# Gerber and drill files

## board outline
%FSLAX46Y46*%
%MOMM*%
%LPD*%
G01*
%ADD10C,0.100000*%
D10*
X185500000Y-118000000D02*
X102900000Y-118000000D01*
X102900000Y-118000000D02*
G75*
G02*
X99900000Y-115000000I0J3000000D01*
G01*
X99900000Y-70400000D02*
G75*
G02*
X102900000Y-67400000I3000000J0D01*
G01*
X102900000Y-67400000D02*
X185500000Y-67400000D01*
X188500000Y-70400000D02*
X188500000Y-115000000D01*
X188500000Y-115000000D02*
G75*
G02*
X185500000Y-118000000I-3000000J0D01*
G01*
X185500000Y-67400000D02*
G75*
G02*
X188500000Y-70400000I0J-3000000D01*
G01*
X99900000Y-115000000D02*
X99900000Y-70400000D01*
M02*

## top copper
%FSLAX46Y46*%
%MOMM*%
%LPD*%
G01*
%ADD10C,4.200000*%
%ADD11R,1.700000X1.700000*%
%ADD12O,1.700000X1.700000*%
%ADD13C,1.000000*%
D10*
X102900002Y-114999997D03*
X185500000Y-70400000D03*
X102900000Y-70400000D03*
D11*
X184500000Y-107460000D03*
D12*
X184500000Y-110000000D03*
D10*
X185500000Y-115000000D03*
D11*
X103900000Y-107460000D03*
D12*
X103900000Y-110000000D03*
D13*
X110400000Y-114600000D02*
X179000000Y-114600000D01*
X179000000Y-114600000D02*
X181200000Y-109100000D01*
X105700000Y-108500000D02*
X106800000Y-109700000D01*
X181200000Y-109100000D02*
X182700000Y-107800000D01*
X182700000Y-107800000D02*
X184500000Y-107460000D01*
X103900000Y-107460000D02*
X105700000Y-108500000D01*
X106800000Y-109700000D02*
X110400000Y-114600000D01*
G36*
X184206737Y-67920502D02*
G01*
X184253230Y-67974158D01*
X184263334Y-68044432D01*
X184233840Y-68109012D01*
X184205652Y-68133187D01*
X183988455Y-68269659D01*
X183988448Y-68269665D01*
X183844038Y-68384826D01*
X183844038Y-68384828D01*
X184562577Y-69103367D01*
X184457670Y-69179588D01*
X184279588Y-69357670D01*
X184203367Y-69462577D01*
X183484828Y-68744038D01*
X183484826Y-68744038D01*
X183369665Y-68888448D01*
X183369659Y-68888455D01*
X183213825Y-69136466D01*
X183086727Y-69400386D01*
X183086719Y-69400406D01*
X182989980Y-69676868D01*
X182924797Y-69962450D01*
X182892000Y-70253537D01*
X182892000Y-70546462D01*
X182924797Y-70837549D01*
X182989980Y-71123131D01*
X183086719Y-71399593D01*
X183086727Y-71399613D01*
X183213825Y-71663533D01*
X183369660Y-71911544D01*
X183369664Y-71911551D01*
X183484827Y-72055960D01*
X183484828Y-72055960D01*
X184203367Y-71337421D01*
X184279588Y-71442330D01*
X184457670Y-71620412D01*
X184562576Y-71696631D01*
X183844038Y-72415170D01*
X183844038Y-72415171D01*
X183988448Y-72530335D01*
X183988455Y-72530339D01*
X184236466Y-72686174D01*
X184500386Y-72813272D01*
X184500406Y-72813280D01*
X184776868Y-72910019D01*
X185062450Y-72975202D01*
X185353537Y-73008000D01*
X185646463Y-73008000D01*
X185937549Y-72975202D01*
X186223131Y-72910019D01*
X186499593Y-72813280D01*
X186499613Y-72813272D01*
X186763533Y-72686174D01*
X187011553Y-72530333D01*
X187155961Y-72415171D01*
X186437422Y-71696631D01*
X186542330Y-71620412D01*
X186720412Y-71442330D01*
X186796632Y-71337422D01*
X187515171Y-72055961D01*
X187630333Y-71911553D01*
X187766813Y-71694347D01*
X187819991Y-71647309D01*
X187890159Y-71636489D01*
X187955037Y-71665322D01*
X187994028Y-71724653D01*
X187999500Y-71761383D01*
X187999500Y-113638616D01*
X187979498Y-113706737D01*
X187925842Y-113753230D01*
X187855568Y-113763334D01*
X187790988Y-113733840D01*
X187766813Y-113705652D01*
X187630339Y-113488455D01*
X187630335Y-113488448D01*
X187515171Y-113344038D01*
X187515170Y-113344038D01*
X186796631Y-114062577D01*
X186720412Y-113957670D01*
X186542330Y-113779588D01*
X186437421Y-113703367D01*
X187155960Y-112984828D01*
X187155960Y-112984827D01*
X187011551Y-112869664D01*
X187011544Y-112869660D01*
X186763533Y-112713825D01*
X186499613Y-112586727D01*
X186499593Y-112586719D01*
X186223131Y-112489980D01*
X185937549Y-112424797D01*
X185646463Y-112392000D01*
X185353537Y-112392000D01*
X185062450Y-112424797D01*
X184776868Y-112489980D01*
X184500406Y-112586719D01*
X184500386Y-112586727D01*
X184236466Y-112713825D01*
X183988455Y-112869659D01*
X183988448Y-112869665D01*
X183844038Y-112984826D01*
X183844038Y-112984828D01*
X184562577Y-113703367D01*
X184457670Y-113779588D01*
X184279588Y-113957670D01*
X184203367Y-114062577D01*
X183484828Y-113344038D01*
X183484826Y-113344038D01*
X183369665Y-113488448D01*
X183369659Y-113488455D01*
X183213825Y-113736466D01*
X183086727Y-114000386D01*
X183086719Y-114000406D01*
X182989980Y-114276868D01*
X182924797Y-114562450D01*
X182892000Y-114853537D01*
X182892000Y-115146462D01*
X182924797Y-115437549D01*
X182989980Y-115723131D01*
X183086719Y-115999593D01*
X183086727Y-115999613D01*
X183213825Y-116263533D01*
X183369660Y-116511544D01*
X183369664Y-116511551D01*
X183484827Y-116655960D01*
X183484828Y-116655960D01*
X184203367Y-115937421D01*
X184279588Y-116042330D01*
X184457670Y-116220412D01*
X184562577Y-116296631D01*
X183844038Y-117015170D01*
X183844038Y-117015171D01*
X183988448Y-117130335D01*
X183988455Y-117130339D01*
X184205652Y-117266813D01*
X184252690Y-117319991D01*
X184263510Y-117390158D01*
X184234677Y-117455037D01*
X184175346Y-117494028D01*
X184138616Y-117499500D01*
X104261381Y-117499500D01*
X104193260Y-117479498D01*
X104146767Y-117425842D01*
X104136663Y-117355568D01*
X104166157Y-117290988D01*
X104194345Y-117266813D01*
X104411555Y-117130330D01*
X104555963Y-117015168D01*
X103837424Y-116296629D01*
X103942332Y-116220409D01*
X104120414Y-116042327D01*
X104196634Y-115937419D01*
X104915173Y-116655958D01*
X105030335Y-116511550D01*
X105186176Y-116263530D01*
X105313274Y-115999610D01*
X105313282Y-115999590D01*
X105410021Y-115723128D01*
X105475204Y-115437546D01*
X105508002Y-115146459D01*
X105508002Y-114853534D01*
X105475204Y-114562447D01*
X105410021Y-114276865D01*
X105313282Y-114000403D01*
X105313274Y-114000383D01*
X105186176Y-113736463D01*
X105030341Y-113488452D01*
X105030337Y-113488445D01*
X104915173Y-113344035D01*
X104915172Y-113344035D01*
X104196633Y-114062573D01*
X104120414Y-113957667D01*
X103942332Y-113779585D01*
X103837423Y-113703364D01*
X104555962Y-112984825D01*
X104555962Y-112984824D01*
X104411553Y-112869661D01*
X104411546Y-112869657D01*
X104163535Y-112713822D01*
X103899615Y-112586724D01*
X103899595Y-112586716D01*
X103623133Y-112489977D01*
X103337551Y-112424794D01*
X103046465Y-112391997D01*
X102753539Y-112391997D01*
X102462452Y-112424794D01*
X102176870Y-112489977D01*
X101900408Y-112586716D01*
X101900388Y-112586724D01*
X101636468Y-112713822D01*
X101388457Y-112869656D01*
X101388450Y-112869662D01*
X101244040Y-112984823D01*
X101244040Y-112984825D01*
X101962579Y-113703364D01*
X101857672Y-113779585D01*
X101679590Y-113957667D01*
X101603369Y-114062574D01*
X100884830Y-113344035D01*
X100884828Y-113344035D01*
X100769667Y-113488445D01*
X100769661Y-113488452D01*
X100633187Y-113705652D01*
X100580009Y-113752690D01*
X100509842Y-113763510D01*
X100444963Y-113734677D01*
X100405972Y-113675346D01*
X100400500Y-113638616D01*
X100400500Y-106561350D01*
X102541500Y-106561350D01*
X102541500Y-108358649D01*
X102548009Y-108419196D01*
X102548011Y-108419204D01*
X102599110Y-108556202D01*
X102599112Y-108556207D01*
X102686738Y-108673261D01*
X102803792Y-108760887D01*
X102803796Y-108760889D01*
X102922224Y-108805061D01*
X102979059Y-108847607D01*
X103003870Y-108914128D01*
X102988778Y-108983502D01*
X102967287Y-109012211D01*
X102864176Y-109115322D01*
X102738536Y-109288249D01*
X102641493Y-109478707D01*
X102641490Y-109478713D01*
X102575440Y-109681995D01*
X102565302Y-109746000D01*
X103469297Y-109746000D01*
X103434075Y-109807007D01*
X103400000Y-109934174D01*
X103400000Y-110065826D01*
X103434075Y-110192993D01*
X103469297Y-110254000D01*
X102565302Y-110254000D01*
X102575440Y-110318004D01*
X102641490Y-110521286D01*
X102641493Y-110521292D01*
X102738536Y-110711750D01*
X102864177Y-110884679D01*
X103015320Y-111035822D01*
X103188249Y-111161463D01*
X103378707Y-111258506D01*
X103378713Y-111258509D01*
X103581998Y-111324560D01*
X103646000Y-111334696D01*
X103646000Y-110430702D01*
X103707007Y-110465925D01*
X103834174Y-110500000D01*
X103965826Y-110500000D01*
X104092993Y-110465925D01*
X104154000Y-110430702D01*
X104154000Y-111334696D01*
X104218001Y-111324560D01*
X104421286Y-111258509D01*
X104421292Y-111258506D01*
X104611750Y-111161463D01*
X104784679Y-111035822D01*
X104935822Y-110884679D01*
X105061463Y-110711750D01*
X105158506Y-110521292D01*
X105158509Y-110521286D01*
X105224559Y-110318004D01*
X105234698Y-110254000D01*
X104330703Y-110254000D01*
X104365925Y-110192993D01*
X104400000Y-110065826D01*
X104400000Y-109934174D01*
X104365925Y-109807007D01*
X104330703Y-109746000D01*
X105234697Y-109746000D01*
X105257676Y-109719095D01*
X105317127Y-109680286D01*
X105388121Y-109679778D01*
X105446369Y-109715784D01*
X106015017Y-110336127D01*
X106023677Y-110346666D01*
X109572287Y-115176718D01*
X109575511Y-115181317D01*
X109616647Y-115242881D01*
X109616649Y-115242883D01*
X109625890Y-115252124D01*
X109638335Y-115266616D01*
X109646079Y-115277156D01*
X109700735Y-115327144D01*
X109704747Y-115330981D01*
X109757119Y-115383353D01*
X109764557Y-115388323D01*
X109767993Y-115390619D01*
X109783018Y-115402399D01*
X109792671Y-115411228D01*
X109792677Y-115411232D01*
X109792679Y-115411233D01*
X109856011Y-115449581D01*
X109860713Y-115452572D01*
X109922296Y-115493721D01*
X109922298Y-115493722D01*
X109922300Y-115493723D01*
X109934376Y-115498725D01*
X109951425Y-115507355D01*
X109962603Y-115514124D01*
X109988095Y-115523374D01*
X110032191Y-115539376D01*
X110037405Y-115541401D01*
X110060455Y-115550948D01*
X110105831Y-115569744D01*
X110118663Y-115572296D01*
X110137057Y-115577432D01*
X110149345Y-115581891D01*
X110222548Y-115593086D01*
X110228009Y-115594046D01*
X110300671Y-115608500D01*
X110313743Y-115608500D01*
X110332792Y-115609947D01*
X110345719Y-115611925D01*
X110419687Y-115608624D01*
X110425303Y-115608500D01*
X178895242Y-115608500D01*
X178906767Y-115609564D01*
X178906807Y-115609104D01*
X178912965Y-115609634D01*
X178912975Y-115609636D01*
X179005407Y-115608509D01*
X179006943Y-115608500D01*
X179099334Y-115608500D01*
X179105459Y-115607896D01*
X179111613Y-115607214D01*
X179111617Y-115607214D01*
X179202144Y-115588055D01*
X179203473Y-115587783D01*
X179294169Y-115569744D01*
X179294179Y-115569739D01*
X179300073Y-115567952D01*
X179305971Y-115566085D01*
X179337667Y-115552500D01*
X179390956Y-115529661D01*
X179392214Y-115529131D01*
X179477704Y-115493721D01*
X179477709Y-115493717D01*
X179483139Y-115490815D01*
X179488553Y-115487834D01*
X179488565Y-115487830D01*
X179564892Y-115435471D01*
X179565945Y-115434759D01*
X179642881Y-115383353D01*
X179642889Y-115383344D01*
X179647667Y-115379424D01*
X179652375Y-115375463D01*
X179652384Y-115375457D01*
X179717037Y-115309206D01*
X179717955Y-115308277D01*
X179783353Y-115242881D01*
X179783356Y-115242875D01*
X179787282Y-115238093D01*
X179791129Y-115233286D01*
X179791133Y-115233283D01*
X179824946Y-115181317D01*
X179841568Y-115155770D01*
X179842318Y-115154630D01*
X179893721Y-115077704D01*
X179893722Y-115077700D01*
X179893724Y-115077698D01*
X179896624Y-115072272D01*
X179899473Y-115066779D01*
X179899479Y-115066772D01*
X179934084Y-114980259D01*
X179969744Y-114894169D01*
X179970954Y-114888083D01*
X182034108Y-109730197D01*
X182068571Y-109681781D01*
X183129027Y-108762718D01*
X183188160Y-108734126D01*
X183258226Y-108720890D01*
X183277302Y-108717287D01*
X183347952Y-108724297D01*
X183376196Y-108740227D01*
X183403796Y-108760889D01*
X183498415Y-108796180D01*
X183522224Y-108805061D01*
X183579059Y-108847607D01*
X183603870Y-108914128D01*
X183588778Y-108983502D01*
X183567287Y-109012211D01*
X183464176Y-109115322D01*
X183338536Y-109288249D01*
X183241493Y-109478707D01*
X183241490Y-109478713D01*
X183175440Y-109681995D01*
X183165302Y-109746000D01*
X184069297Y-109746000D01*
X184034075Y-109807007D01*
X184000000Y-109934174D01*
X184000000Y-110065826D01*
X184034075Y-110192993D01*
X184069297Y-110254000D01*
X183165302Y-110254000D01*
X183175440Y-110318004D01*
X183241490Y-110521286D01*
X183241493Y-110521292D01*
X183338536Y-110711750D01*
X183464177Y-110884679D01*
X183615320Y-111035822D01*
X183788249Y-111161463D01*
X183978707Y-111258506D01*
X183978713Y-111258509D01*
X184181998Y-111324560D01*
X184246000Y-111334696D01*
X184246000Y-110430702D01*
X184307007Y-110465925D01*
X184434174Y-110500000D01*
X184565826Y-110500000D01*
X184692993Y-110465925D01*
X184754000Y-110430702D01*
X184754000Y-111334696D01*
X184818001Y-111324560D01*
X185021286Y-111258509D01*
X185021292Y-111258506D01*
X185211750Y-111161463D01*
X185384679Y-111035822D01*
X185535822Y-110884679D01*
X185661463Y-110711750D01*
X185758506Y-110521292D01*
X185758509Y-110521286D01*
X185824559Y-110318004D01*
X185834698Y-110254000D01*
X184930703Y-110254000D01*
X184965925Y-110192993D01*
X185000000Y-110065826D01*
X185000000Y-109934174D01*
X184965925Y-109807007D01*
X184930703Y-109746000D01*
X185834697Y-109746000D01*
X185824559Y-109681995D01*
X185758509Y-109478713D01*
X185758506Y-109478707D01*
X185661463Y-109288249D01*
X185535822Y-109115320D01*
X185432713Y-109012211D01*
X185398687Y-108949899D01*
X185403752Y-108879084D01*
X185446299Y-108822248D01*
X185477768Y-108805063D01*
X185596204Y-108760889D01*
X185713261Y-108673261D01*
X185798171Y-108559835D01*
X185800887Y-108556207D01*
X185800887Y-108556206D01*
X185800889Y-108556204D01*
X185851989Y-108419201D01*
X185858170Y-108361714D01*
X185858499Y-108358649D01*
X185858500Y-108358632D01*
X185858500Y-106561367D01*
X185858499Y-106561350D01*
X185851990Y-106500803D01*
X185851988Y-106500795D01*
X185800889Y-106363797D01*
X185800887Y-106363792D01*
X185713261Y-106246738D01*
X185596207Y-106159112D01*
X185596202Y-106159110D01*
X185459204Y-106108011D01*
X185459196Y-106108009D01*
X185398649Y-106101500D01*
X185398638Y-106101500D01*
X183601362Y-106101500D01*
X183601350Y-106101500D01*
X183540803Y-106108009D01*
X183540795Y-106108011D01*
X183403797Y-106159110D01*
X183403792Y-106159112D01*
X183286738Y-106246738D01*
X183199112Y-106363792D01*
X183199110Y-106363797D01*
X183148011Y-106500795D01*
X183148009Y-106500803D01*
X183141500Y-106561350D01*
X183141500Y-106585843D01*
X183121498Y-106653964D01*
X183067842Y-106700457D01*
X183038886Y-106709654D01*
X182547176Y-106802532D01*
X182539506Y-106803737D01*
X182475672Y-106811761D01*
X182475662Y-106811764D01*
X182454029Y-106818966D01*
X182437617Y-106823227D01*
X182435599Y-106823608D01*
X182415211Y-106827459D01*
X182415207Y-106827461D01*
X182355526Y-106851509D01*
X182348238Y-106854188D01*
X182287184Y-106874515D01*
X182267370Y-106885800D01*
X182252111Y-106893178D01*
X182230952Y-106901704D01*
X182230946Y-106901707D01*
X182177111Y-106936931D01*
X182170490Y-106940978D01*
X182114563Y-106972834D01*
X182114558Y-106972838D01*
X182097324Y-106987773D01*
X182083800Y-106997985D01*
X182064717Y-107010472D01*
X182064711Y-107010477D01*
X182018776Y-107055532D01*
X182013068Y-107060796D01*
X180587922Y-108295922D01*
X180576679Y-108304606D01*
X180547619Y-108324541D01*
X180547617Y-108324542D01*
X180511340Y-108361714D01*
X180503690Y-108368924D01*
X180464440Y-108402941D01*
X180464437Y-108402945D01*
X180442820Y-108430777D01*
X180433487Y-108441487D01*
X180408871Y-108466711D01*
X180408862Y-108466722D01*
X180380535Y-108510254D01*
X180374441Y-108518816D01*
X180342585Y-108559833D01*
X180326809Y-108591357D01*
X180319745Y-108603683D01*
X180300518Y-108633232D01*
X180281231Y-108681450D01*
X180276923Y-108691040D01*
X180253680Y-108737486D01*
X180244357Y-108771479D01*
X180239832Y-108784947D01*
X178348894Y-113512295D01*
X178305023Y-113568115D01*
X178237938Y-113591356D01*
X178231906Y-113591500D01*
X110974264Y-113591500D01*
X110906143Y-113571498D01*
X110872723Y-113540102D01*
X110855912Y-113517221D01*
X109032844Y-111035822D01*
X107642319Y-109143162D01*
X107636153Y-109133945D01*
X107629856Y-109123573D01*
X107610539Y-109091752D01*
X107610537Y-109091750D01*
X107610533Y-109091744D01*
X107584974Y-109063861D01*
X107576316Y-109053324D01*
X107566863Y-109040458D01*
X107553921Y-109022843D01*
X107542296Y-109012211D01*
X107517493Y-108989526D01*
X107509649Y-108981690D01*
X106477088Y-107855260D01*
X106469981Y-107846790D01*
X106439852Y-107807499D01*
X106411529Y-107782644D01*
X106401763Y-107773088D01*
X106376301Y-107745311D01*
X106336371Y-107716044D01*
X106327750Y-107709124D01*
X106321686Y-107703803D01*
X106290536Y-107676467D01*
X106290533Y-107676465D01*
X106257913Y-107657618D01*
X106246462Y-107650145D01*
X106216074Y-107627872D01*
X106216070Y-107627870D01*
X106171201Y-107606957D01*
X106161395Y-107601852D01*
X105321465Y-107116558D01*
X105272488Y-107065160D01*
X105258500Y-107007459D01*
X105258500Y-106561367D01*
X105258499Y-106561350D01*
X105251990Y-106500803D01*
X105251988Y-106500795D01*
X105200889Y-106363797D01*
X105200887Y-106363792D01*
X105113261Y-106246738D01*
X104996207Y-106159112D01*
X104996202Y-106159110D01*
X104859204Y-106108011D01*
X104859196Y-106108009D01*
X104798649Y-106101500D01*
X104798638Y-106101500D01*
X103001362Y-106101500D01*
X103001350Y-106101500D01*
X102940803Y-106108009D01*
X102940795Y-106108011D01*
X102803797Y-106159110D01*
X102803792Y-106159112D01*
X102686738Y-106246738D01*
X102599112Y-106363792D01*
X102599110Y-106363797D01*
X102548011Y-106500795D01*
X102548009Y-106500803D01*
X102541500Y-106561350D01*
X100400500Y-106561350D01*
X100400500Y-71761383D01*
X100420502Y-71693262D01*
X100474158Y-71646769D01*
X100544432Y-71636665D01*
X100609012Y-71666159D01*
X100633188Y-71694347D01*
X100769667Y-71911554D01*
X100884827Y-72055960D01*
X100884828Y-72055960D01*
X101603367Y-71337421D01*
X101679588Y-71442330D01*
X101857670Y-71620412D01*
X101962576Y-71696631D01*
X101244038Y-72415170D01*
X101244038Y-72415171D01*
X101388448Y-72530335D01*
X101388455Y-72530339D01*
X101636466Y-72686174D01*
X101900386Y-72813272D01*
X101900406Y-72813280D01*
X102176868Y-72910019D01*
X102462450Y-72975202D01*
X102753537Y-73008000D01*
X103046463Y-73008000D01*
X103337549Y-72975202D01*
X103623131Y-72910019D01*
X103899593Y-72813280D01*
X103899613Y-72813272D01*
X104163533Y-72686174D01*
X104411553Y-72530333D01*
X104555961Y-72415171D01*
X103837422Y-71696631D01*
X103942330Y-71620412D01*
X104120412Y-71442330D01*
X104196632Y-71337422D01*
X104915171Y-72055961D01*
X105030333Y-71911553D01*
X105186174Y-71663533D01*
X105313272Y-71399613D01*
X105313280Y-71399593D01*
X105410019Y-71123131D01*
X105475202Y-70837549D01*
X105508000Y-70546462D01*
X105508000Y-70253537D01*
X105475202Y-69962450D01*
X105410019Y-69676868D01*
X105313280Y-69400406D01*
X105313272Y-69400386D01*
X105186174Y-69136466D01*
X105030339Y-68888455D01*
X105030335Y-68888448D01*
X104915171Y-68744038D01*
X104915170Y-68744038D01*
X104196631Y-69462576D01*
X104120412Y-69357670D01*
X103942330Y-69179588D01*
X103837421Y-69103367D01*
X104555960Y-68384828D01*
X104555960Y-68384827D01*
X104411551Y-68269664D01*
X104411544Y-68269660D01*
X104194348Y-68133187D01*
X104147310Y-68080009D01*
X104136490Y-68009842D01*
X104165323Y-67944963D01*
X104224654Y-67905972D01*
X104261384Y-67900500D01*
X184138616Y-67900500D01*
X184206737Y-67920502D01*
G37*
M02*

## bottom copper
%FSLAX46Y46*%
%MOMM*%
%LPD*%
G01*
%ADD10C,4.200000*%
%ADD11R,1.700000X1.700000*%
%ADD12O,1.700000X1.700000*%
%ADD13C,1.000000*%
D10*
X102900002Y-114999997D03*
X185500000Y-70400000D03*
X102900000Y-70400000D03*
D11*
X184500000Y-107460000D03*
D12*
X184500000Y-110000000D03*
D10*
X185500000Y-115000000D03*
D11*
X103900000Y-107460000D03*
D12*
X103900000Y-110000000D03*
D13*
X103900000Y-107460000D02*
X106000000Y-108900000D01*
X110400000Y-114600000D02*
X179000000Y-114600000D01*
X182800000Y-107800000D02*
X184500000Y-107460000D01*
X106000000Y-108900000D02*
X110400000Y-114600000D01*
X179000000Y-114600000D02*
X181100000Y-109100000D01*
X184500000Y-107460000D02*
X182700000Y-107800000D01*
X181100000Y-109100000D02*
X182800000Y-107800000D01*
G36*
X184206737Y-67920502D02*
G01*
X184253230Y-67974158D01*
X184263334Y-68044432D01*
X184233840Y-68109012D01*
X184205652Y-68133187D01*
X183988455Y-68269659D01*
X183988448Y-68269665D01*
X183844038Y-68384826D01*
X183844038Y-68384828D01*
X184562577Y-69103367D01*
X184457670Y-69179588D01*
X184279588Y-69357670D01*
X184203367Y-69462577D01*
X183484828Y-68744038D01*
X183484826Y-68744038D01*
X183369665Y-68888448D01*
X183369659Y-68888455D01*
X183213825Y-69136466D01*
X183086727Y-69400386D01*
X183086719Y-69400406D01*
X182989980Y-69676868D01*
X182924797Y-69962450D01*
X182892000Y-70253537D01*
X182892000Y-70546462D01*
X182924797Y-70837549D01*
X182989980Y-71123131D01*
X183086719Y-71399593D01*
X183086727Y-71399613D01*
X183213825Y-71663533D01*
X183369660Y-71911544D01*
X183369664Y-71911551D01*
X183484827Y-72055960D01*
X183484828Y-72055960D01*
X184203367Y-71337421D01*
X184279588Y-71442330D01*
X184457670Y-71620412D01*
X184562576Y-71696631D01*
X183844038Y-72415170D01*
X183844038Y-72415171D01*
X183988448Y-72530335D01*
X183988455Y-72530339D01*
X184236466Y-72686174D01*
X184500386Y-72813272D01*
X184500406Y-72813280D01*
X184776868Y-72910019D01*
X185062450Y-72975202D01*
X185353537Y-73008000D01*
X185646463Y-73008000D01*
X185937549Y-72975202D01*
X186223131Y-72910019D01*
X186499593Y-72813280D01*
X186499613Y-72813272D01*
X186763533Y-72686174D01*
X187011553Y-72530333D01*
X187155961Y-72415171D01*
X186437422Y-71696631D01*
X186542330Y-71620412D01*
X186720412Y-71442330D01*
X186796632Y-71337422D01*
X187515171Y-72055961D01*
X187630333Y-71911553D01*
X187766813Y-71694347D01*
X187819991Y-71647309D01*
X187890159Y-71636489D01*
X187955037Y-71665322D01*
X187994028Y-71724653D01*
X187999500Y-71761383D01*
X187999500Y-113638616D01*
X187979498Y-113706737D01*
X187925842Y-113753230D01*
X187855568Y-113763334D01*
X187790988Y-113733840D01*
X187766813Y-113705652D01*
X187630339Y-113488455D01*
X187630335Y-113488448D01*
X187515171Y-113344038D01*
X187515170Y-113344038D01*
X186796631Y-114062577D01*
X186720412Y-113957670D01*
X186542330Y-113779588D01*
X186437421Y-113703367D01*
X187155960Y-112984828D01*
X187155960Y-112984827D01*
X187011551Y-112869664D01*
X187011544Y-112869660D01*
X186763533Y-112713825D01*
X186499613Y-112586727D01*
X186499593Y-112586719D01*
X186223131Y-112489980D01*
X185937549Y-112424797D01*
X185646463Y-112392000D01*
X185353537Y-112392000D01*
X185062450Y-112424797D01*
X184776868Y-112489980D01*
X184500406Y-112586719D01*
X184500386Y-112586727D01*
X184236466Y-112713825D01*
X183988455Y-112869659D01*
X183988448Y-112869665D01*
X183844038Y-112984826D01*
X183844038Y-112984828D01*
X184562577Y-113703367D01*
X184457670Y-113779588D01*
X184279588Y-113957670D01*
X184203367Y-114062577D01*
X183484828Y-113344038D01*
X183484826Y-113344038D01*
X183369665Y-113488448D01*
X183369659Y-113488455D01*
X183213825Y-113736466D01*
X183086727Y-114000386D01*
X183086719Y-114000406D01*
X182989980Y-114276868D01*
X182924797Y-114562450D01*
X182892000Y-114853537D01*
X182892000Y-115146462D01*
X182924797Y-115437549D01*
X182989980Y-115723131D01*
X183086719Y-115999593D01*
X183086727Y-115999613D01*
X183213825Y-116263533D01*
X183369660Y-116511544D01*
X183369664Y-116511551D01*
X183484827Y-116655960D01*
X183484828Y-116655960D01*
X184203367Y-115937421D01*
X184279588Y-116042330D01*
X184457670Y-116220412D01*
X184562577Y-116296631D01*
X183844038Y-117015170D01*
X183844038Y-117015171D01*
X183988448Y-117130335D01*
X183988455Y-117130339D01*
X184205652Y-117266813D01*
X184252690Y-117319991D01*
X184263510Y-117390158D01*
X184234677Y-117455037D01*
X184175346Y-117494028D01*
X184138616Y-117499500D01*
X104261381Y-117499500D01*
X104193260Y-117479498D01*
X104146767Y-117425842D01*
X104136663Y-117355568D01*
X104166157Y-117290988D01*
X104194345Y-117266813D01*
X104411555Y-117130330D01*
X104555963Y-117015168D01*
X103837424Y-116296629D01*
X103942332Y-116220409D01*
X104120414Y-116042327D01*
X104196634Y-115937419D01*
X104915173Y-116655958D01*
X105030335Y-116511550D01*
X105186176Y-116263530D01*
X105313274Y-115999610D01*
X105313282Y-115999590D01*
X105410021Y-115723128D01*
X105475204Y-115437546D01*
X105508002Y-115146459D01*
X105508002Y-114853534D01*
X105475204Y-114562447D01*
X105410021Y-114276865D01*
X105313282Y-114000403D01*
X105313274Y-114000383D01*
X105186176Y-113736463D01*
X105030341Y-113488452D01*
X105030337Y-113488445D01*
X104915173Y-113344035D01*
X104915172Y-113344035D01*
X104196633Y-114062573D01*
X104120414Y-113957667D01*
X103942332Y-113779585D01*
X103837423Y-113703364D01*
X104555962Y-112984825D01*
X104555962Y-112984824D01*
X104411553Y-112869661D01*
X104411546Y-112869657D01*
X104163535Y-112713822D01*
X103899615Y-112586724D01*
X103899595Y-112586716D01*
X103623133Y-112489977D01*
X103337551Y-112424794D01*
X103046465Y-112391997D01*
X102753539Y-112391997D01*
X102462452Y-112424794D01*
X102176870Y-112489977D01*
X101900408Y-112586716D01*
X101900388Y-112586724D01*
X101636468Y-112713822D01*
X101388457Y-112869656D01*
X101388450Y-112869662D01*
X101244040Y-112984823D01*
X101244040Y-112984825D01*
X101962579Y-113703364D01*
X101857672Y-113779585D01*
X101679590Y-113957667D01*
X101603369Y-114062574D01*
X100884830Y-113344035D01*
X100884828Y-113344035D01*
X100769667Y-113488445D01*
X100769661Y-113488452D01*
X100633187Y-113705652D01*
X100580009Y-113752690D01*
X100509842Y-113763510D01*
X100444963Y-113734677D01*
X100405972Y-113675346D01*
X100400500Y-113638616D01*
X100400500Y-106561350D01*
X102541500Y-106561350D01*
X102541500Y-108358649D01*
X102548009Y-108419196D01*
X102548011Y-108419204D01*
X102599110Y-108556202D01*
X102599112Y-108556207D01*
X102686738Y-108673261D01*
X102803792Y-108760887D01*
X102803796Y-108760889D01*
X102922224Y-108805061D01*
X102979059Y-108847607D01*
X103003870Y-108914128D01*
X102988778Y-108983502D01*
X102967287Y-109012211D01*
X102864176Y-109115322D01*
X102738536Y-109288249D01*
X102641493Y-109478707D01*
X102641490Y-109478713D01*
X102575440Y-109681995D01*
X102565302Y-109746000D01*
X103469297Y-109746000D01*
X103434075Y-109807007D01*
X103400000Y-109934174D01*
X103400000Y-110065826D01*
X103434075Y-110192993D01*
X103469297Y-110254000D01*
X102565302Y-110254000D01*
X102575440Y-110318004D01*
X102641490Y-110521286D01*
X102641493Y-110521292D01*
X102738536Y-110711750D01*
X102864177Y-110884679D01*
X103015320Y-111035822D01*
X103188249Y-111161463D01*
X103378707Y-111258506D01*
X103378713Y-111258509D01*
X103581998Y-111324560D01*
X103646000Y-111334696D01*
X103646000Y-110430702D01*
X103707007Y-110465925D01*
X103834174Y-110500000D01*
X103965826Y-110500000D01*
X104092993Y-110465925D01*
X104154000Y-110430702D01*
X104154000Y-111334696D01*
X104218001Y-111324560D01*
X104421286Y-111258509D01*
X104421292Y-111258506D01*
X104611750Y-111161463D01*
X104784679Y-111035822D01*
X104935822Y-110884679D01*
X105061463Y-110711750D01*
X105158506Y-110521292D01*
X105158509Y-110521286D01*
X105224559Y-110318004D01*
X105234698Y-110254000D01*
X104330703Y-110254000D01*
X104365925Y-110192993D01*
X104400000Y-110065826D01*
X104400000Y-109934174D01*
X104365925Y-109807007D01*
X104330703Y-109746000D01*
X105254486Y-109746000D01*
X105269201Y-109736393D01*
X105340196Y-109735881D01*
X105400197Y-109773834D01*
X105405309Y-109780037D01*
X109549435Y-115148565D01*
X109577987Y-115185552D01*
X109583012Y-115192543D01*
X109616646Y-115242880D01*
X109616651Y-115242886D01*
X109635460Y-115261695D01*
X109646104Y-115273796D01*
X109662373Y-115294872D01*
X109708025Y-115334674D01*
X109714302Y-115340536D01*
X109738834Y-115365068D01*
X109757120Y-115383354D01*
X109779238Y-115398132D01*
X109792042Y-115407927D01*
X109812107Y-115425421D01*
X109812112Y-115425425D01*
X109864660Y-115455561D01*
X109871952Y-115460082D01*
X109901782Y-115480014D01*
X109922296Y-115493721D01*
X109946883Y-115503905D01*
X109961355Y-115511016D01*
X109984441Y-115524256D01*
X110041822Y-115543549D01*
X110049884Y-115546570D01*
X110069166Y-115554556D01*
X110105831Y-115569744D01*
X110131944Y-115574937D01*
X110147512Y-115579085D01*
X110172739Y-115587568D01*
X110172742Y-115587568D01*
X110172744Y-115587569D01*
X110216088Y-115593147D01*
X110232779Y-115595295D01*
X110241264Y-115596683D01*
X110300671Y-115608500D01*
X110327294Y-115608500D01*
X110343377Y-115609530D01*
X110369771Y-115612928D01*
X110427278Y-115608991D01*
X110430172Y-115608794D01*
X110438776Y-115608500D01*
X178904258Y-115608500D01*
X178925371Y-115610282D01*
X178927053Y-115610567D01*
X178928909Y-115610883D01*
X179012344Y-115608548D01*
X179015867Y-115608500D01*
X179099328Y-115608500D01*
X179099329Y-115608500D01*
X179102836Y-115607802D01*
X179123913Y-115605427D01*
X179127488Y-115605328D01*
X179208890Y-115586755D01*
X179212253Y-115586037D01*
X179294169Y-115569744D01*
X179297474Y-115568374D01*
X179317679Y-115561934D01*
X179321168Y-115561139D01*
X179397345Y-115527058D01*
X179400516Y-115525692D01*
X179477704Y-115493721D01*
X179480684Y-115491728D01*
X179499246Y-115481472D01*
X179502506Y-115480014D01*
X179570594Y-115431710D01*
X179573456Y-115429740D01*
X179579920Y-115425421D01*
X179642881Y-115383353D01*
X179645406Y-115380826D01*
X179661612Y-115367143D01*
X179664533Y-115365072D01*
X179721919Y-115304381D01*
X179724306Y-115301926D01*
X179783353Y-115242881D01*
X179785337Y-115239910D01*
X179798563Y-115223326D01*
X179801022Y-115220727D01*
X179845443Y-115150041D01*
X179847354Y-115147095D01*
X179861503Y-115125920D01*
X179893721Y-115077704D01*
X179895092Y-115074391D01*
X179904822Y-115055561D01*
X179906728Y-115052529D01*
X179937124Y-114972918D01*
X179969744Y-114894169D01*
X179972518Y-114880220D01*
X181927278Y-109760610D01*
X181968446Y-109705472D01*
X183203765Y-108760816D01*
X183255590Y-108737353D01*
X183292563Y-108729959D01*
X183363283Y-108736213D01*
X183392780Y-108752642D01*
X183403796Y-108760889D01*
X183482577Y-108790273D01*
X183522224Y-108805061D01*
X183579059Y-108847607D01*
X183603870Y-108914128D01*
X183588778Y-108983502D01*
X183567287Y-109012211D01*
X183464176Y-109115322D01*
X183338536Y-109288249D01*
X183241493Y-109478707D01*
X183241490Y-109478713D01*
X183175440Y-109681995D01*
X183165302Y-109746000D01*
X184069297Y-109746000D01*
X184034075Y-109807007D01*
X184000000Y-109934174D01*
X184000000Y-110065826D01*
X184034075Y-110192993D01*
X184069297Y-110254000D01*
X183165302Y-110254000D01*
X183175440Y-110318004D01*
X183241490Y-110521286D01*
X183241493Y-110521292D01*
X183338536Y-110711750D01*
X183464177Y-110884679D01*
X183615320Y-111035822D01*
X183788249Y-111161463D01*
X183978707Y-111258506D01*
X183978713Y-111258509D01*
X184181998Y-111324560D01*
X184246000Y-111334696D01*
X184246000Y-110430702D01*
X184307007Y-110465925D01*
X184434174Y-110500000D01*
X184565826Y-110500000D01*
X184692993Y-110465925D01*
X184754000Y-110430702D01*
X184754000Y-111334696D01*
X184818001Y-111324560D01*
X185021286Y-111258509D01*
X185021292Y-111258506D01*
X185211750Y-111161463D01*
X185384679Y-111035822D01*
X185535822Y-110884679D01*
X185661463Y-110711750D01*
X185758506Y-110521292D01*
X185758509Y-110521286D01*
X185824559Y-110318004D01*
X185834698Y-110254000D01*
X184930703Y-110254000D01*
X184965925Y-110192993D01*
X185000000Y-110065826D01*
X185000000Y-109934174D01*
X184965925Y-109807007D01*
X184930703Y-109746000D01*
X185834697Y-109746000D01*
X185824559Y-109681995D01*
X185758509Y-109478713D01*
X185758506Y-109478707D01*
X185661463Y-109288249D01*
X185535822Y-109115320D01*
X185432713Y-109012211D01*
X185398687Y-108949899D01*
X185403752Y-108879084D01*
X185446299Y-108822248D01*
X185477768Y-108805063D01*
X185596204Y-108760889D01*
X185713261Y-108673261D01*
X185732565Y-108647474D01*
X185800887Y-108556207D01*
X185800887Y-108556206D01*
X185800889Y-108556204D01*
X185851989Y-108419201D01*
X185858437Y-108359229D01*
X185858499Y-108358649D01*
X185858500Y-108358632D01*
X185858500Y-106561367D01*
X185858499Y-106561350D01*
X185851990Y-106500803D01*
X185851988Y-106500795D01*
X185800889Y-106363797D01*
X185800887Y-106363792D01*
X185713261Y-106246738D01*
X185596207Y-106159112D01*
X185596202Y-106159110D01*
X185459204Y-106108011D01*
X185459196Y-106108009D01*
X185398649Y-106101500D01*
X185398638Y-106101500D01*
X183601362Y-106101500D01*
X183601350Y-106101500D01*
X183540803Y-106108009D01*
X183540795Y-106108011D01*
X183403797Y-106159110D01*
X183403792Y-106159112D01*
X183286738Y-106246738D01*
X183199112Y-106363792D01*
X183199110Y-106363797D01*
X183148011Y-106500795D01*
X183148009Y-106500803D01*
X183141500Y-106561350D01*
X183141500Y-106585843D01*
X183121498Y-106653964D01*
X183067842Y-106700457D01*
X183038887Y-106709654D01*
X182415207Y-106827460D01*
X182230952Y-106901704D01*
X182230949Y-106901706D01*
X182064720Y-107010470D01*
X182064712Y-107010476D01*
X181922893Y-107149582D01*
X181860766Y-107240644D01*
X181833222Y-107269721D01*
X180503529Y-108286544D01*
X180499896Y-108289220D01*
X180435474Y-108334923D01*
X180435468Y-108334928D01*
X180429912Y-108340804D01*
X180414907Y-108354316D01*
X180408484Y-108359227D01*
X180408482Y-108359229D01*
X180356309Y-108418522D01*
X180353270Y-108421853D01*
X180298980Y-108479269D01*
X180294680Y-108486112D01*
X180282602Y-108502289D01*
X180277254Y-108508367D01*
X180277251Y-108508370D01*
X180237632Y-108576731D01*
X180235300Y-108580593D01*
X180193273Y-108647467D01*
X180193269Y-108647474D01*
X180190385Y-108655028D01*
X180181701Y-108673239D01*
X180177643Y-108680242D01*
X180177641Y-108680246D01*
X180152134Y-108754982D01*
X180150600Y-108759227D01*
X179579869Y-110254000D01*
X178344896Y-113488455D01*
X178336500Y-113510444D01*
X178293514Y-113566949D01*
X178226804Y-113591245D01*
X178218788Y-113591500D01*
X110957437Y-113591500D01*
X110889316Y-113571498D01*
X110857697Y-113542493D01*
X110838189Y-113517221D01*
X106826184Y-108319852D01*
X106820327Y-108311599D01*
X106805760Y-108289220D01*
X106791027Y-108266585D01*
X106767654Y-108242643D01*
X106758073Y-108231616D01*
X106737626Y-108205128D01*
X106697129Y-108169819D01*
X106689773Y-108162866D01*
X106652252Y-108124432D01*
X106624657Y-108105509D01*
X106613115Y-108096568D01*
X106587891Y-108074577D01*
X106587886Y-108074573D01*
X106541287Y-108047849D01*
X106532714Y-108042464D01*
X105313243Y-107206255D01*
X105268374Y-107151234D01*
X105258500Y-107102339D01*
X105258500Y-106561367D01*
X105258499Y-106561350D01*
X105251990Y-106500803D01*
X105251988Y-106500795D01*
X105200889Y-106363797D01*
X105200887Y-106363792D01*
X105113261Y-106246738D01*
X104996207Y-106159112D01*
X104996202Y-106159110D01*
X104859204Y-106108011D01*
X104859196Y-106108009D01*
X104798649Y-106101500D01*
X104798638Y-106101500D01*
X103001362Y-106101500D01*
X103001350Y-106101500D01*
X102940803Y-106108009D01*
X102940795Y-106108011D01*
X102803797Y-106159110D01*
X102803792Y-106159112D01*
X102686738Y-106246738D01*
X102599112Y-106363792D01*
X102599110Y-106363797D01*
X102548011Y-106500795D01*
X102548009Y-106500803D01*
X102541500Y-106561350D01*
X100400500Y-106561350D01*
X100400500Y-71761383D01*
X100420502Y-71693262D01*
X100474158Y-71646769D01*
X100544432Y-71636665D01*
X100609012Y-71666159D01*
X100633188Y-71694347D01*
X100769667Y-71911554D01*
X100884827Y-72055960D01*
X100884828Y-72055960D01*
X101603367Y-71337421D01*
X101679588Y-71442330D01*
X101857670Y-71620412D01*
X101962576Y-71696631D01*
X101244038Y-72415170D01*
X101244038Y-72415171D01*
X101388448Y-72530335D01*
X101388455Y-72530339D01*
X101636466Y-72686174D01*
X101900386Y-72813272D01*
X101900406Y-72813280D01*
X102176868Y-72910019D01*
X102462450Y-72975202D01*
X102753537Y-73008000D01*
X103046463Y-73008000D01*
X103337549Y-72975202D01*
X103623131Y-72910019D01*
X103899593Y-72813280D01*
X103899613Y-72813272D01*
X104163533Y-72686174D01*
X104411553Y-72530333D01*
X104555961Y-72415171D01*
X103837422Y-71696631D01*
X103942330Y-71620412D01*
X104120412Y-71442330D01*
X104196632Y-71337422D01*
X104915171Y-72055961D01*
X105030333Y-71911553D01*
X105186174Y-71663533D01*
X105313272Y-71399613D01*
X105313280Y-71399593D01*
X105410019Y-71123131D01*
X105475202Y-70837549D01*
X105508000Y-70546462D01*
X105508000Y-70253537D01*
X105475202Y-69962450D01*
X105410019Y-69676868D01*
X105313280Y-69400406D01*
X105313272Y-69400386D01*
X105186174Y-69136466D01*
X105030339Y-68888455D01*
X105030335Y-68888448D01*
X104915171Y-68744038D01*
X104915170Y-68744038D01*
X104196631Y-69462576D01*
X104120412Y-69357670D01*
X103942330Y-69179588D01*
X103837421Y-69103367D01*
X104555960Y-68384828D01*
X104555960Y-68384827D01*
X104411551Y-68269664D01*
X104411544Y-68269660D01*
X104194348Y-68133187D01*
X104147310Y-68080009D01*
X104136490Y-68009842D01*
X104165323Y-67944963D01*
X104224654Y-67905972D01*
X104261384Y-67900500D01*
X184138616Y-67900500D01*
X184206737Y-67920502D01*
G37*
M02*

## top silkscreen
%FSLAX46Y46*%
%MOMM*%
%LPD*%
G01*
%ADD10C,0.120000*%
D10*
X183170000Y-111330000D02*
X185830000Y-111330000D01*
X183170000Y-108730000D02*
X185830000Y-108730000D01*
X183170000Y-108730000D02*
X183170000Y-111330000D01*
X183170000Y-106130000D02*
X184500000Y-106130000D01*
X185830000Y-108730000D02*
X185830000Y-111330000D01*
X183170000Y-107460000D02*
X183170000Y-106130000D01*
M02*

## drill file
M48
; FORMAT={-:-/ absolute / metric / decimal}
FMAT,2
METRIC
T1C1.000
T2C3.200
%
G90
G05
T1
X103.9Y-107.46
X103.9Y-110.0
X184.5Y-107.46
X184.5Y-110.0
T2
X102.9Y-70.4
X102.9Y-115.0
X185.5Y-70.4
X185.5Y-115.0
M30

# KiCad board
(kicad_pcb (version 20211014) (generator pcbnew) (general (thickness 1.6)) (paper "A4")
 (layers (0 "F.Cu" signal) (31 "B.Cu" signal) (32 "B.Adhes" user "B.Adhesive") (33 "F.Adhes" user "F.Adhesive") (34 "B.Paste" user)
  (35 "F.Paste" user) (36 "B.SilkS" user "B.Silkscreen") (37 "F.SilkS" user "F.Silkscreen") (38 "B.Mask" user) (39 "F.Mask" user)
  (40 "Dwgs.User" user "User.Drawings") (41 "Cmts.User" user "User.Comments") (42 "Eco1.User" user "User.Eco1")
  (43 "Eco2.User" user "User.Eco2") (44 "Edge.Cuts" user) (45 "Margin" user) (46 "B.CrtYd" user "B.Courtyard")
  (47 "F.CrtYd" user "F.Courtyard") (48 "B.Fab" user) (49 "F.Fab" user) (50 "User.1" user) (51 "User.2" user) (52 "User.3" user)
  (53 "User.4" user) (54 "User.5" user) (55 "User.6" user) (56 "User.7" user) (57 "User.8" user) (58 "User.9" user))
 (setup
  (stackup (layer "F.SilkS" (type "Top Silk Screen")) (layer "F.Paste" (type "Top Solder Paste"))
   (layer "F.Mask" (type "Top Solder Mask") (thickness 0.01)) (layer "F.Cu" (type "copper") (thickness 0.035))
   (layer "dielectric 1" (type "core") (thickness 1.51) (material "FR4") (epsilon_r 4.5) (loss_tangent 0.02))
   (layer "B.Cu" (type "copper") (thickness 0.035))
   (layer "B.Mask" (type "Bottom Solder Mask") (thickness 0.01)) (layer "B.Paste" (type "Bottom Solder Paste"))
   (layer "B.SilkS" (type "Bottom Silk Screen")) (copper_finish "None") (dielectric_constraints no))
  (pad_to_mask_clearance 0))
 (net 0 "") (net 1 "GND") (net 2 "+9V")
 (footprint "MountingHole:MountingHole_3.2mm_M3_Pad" (layer "F.Cu") (at 102.900002 114.999997)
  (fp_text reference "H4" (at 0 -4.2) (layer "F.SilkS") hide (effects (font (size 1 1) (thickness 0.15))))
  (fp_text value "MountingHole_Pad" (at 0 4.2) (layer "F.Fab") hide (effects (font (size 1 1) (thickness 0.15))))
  (pad "1" thru_hole circle (at 0 0) (size 4.2 4.2) (drill 3.2) (layers *.Cu *.Mask) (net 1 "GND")))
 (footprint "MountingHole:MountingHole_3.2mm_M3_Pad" (layer "F.Cu") (at 185.5 70.4)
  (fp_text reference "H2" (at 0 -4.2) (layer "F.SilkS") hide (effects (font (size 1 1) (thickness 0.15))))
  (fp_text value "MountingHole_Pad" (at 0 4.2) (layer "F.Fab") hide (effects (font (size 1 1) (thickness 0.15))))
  (pad "1" thru_hole circle (at 0 0) (size 4.2 4.2) (drill 3.2) (layers *.Cu *.Mask) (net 1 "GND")))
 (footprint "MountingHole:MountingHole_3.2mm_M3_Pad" (layer "F.Cu") (at 102.9 70.4)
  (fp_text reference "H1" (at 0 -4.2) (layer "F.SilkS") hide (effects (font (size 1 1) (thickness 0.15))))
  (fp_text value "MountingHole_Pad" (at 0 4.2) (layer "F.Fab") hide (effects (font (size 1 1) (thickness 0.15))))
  (pad "1" thru_hole circle (at 0 0) (size 4.2 4.2) (drill 3.2) (layers *.Cu *.Mask) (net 1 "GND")))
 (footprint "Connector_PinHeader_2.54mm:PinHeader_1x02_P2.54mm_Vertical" (layer "F.Cu") (at 184.5 107.46)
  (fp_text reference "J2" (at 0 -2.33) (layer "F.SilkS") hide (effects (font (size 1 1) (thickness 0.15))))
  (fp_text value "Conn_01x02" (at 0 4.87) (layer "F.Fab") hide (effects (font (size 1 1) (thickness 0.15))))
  (fp_line (start -1.33 3.87) (end 1.33 3.87) (layer "F.SilkS") (width 0.12))
  (fp_line (start -1.33 1.27) (end 1.33 1.27) (layer "F.SilkS") (width 0.12))
  (fp_line (start -1.33 1.27) (end -1.33 3.87) (layer "F.SilkS") (width 0.12))
  (fp_line (start -1.33 -1.33) (end 0 -1.33) (layer "F.SilkS") (width 0.12))
  (fp_line (start 1.33 1.27) (end 1.33 3.87) (layer "F.SilkS") (width 0.12))
  (fp_line (start -1.33 0) (end -1.33 -1.33) (layer "F.SilkS") (width 0.12))
  (pad "1" thru_hole rect (at 0 0) (size 1.7 1.7) (drill 1) (layers *.Cu *.Mask) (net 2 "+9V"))
  (pad "2" thru_hole oval (at 0 2.54) (size 1.7 1.7) (drill 1) (layers *.Cu *.Mask) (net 1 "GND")))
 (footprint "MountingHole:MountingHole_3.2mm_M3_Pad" (layer "F.Cu") (at 185.5 115)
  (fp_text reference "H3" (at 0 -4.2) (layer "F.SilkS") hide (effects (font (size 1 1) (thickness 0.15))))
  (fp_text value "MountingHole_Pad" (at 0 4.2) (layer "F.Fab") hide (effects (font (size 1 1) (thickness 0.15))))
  (pad "1" thru_hole circle (at 0 0) (size 4.2 4.2) (drill 3.2) (layers *.Cu *.Mask) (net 1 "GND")))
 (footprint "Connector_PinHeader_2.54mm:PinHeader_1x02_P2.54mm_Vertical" (layer "B.Cu") (at 103.9 107.46 180)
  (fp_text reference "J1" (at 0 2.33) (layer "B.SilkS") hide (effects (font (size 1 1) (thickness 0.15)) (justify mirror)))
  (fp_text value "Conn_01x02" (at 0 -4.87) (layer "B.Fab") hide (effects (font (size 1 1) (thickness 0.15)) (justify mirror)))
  (pad "1" thru_hole rect (at 0 0 180) (size 1.7 1.7) (drill 1) (layers *.Cu *.Mask) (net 2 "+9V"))
  (pad "2" thru_hole oval (at 0 -2.54 180) (size 1.7 1.7) (drill 1) (layers *.Cu *.Mask) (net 1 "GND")))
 (gr_line (start 185.5 118) (end 102.9 118) (layer "Edge.Cuts") (width 0.1))
 (gr_arc (start 102.9 118) (mid 100.77868 117.12132) (end 99.9 115) (layer "Edge.Cuts") (width 0.1))
 (gr_arc (start 99.9 70.4) (mid 100.778681 68.278681) (end 102.9 67.4) (layer "Edge.Cuts") (width 0.1))
 (gr_line (start 102.9 67.4) (end 185.5 67.4) (layer "Edge.Cuts") (width 0.1))
 (gr_line (start 188.5 70.4) (end 188.5 115) (layer "Edge.Cuts") (width 0.1))
 (gr_arc (start 188.5 115) (mid 187.62132 117.12132) (end 185.5 118) (layer "Edge.Cuts") (width 0.1))
 (gr_arc (start 185.5 67.4) (mid 187.621319 68.278681) (end 188.5 70.4) (layer "Edge.Cuts") (width 0.1))
 (gr_line (start 99.9 115) (end 99.9 70.4) (layer "Edge.Cuts") (width 0.1))
 (segment (start 110.4 114.6) (end 179 114.6) (width 1) (layer "F.Cu") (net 2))
 (segment (start 179 114.6) (end 181.2 109.1) (width 1) (layer "F.Cu") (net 2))
 (segment (start 105.7 108.5) (end 106.8 109.7) (width 1) (layer "F.Cu") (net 2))
 (segment (start 181.2 109.1) (end 182.7 107.8) (width 1) (layer "F.Cu") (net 2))
 (segment (start 182.7 107.8) (end 184.5 107.46) (width 1) (layer "F.Cu") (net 2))
 (segment (start 103.9 107.46) (end 105.7 108.5) (width 1) (layer "F.Cu") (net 2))
 (segment (start 106.8 109.7) (end 110.4 114.6) (width 1) (layer "F.Cu") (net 2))
 (segment (start 103.9 107.46) (end 106 108.9) (width 1) (layer "B.Cu") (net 2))
 (segment (start 110.4 114.6) (end 179 114.6) (width 1) (layer "B.Cu") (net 2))
 (segment (start 182.8 107.8) (end 184.5 107.46) (width 1) (layer "B.Cu") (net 2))
 (segment (start 106 108.9) (end 110.4 114.6) (width 1) (layer "B.Cu") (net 2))
 (segment (start 179 114.6) (end 181.1 109.1) (width 1) (layer "B.Cu") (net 2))
 (segment (start 184.5 107.46) (end 182.7 107.8) (width 1) (layer "B.Cu") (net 2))
 (segment (start 181.1 109.1) (end 182.8 107.8) (width 1) (layer "B.Cu") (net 2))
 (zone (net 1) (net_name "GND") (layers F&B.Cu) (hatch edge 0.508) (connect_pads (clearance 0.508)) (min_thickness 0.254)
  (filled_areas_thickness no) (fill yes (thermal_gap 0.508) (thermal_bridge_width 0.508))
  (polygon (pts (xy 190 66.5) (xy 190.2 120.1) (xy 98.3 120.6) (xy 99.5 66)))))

